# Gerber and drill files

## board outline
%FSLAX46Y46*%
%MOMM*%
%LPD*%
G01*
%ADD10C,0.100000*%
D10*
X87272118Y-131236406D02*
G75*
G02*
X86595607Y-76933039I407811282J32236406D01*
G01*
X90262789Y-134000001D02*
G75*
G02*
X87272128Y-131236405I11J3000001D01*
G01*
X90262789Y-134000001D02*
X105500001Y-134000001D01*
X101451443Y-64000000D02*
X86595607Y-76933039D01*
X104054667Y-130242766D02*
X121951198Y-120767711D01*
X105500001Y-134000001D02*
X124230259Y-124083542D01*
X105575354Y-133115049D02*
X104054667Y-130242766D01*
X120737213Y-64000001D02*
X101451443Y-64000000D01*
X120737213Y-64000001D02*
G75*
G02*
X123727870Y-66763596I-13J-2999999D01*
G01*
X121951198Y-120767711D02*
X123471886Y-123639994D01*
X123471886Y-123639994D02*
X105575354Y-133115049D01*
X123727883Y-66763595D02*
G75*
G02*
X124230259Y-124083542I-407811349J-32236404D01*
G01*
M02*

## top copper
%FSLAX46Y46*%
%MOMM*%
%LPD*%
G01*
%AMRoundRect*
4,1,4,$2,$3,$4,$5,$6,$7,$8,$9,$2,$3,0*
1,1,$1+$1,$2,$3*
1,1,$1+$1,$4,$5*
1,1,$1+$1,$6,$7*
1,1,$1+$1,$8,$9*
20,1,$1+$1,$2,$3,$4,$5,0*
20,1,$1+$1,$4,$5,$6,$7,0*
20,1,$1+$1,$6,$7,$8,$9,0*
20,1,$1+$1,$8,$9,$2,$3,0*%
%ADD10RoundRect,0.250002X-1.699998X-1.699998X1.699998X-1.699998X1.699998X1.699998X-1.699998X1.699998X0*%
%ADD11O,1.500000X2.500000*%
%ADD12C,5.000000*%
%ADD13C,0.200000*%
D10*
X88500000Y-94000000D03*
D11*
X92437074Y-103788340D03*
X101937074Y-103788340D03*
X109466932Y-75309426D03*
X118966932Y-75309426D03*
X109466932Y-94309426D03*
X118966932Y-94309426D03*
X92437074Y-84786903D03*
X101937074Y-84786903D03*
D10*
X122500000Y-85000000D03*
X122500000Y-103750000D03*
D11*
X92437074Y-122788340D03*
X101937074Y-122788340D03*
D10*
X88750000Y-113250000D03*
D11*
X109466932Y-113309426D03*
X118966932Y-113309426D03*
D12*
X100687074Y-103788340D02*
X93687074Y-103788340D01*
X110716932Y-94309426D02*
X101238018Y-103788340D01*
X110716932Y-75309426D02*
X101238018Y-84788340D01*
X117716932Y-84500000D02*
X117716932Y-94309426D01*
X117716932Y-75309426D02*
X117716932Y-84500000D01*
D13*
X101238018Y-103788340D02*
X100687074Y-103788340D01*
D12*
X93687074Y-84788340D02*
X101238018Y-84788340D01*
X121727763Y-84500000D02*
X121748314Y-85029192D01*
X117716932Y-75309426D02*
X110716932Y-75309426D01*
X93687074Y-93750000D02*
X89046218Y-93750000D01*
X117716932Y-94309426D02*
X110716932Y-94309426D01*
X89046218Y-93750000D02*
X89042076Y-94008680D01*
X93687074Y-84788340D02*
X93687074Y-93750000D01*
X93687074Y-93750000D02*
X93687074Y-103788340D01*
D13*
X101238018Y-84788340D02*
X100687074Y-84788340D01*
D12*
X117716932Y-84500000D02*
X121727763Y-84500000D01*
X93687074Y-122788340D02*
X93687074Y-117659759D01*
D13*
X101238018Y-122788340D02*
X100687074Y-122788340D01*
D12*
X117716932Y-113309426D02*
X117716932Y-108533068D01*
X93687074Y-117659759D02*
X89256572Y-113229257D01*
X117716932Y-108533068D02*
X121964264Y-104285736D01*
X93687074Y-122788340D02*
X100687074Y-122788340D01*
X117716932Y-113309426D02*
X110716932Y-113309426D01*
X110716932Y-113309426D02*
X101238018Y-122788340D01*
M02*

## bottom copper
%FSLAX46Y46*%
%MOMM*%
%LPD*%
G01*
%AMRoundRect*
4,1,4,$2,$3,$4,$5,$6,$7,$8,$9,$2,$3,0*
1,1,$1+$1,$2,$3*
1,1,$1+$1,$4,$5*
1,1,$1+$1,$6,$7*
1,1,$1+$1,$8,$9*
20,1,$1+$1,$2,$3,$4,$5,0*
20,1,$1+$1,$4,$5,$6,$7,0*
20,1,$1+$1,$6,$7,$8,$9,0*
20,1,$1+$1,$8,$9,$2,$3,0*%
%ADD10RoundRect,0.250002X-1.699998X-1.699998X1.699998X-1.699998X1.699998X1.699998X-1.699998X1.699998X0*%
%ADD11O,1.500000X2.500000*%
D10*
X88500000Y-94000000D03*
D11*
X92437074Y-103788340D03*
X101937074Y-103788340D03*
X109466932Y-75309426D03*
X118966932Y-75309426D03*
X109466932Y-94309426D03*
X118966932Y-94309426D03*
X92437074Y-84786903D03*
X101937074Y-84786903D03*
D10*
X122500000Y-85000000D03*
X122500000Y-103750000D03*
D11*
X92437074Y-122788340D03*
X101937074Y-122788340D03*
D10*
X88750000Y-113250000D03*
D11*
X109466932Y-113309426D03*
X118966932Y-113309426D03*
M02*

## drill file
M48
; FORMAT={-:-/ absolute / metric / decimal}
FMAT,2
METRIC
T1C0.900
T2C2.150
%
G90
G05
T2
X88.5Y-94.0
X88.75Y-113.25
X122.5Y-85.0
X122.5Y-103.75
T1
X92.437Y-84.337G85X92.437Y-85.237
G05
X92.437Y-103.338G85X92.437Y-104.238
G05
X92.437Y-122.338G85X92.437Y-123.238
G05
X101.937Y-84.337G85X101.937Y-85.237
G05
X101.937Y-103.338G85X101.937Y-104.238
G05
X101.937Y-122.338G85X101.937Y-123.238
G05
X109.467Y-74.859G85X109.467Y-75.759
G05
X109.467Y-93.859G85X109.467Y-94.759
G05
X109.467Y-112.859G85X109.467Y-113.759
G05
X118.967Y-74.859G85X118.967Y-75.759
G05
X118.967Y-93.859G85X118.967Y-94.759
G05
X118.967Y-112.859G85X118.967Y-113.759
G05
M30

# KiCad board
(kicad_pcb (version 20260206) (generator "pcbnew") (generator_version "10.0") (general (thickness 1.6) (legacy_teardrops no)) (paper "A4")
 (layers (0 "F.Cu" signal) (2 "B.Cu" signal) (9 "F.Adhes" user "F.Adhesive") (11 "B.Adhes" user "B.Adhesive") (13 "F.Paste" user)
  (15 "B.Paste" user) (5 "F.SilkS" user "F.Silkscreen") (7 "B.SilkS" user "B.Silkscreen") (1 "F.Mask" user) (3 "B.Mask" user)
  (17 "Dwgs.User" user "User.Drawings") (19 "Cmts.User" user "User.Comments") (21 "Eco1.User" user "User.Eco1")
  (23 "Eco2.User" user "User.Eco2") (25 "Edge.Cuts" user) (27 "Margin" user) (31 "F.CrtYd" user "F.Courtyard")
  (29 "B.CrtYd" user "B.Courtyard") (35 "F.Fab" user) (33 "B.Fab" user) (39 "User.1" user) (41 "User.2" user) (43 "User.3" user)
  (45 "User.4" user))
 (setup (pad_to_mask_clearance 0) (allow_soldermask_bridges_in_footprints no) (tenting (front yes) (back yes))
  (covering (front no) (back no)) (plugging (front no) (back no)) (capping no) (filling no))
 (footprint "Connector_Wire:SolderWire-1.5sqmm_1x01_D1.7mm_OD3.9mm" (layer "F.Cu") (at 88.5 94)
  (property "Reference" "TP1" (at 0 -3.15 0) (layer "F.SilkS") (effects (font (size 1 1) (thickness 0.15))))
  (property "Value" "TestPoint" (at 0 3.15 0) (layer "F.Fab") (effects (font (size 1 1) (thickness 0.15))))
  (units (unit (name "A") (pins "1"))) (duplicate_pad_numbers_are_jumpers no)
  (pad "1" thru_hole roundrect (at 0 0) (size 3.9 3.9) (drill 2.15) (layers "*.Cu" "*.Mask") (remove_unused_layers no)
   (roundrect_rratio 0.064103) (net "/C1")))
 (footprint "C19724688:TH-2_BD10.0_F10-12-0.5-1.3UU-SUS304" (layer "F.Cu") (at 97.187074 103.78834)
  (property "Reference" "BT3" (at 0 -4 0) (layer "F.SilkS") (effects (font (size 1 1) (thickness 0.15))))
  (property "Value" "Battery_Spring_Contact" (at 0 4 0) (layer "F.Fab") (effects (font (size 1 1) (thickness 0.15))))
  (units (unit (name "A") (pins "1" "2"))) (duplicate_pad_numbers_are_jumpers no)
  (pad "1" thru_hole oval (at -4.75 0) (size 1.5 2.5) (drill oval 0.900024 1.799996) (layers "*.Cu" "*.Mask") (remove_unused_layers no)
   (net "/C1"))
  (pad "2" thru_hole oval (at 4.75 0) (size 1.5 2.5) (drill oval 0.900024 1.799996) (layers "*.Cu" "*.Mask") (remove_unused_layers no)
   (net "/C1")))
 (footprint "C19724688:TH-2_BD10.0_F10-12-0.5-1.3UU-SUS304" (layer "F.Cu") (at 114.216932 75.309426)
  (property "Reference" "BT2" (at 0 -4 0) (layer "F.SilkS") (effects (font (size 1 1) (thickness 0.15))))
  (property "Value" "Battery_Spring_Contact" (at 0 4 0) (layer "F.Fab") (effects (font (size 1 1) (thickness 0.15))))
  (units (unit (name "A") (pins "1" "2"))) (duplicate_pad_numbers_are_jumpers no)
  (pad "1" thru_hole oval (at -4.75 0) (size 1.5 2.5) (drill oval 0.900024 1.799996) (layers "*.Cu" "*.Mask") (remove_unused_layers no)
   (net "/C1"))
  (pad "2" thru_hole oval (at 4.75 0) (size 1.5 2.5) (drill oval 0.900024 1.799996) (layers "*.Cu" "*.Mask") (remove_unused_layers no)
   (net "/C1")))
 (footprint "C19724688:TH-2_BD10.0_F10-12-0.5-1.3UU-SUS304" (layer "F.Cu") (at 114.216932 94.309426)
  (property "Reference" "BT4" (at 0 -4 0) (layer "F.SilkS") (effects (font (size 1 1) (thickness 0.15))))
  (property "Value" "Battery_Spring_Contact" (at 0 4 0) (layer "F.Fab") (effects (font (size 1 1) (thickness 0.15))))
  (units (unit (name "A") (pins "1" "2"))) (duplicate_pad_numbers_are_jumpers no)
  (pad "1" thru_hole oval (at -4.75 0) (size 1.5 2.5) (drill oval 0.900024 1.799996) (layers "*.Cu" "*.Mask") (remove_unused_layers no)
   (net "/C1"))
  (pad "2" thru_hole oval (at 4.75 0) (size 1.5 2.5) (drill oval 0.900024 1.799996) (layers "*.Cu" "*.Mask") (remove_unused_layers no)
   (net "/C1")))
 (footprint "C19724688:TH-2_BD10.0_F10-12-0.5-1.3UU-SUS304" (layer "F.Cu") (at 97.187074 84.786903)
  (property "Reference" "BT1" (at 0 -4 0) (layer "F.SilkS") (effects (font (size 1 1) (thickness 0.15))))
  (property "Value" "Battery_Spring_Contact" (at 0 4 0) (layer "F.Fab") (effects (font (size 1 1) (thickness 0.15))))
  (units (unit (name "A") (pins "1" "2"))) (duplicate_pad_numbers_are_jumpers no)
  (pad "1" thru_hole oval (at -4.75 0) (size 1.5 2.5) (drill oval 0.900024 1.799996) (layers "*.Cu" "*.Mask") (remove_unused_layers no)
   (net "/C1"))
  (pad "2" thru_hole oval (at 4.75 0) (size 1.5 2.5) (drill oval 0.900024 1.799996) (layers "*.Cu" "*.Mask") (remove_unused_layers no)
   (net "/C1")))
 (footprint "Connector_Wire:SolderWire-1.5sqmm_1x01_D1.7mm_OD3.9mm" (layer "F.Cu") (at 122.5 85)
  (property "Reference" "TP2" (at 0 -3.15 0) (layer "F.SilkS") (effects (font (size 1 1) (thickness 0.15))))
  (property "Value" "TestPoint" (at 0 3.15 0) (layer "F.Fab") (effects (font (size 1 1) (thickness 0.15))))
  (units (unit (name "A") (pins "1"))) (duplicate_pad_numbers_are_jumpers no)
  (pad "1" thru_hole roundrect (at 0 0) (size 3.9 3.9) (drill 2.15) (layers "*.Cu" "*.Mask") (remove_unused_layers no)
   (roundrect_rratio 0.064103) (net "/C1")))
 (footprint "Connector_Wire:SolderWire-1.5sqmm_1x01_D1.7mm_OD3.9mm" (layer "F.Cu") (at 122.5 103.75)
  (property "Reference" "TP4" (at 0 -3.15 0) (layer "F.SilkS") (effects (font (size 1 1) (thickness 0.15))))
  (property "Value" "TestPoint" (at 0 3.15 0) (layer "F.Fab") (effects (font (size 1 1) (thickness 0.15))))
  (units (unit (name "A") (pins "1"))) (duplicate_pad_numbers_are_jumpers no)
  (pad "1" thru_hole roundrect (at 0 0) (size 3.9 3.9) (drill 2.15) (layers "*.Cu" "*.Mask") (remove_unused_layers no)
   (roundrect_rratio 0.064103) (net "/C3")))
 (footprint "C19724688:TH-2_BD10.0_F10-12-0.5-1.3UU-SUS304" (layer "F.Cu") (at 97.187074 122.78834)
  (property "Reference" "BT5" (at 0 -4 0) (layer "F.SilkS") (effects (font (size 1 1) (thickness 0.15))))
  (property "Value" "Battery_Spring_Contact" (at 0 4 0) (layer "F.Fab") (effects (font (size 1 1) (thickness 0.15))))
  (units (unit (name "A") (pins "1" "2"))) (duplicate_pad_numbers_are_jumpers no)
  (pad "1" thru_hole oval (at -4.75 0) (size 1.5 2.5) (drill oval 0.900024 1.799996) (layers "*.Cu" "*.Mask") (remove_unused_layers no)
   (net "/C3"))
  (pad "2" thru_hole oval (at 4.75 0) (size 1.5 2.5) (drill oval 0.900024 1.799996) (layers "*.Cu" "*.Mask") (remove_unused_layers no)
   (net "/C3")))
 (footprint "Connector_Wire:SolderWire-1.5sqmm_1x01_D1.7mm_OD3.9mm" (layer "F.Cu") (at 88.75 113.25)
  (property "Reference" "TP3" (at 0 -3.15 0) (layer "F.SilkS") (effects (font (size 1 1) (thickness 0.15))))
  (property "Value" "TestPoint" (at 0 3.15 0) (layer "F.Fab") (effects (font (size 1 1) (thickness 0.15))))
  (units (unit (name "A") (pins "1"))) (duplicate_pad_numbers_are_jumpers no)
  (pad "1" thru_hole roundrect (at 0 0) (size 3.9 3.9) (drill 2.15) (layers "*.Cu" "*.Mask") (remove_unused_layers no)
   (roundrect_rratio 0.064103) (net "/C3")))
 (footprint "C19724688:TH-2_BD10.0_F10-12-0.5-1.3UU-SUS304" (layer "F.Cu") (at 114.216932 113.309426)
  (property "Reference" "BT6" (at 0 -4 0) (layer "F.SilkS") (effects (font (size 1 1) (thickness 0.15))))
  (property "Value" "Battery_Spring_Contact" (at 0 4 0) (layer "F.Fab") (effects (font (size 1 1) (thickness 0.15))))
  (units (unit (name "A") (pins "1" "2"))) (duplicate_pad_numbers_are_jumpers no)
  (pad "1" thru_hole oval (at -4.75 0) (size 1.5 2.5) (drill oval 0.900024 1.799996) (layers "*.Cu" "*.Mask") (remove_unused_layers no)
   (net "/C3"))
  (pad "2" thru_hole oval (at 4.75 0) (size 1.5 2.5) (drill oval 0.900024 1.799996) (layers "*.Cu" "*.Mask") (remove_unused_layers no)
   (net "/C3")))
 (gr_arc (start 87.272118 131.236406) (mid 86.031742 104.095961) (end 86.595607 76.933039) (stroke (width 0.1) (type default))
  (layer "Edge.Cuts"))
 (gr_arc (start 90.262789 134.000001) (mid 88.226767 133.203318) (end 87.272118 131.236406) (stroke (width 0.1) (type default))
  (layer "Edge.Cuts"))
 (gr_line (start 90.262789 134.000001) (end 105.500001 134.000001) (stroke (width 0.1) (type default)) (layer "Edge.Cuts"))
 (gr_line (start 101.451443 64) (end 86.595607 76.933039) (stroke (width 0.1) (type default)) (layer "Edge.Cuts"))
 (gr_line (start 104.054667 130.242766) (end 121.951198 120.767711) (stroke (width 0.1) (type default)) (layer "Edge.Cuts"))
 (gr_line (start 105.500001 134.000001) (end 124.230259 124.083542) (stroke (width 0.1) (type default)) (layer "Edge.Cuts"))
 (gr_line (start 105.575354 133.115049) (end 104.054667 130.242766) (stroke (width 0.1) (type default)) (layer "Edge.Cuts"))
 (gr_line (start 120.737213 64.000001) (end 101.451443 64) (stroke (width 0.1) (type default)) (layer "Edge.Cuts"))
 (gr_arc (start 120.737213 64.000001) (mid 122.773235 64.796684) (end 123.727883 66.763595) (stroke (width 0.1) (type default))
  (layer "Edge.Cuts"))
 (gr_line (start 121.951198 120.767711) (end 123.471886 123.639994) (stroke (width 0.1) (type default)) (layer "Edge.Cuts"))
 (gr_line (start 123.471886 123.639994) (end 105.575354 133.115049) (stroke (width 0.1) (type default)) (layer "Edge.Cuts"))
 (gr_arc (start 123.727883 66.763595) (mid 124.984289 95.414758) (end 124.230259 124.083542) (stroke (width 0.1) (type default))
  (layer "Edge.Cuts"))
 (segment (start 100.687074 103.78834) (end 93.687074 103.78834) (width 5) (layer "F.Cu") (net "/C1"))
 (segment (start 110.716932 94.309426) (end 101.238018 103.78834) (width 5) (layer "F.Cu") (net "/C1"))
 (segment (start 110.716932 75.309426) (end 101.238018 84.78834) (width 5) (layer "F.Cu") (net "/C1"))
 (segment (start 117.716932 84.5) (end 117.716932 94.309426) (width 5) (layer "F.Cu") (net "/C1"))
 (segment (start 117.716932 75.309426) (end 117.716932 84.5) (width 5) (layer "F.Cu") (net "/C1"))
 (segment (start 101.238018 103.78834) (end 100.687074 103.78834) (width 0.2) (layer "F.Cu") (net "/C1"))
 (segment (start 93.687074 84.78834) (end 101.238018 84.78834) (width 5) (layer "F.Cu") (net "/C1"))
 (segment (start 121.727763 84.5) (end 121.748314 85.029192) (width 5) (layer "F.Cu") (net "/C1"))
 (segment (start 117.716932 75.309426) (end 110.716932 75.309426) (width 5) (layer "F.Cu") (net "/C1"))
 (segment (start 93.687074 93.75) (end 89.046218 93.75) (width 5) (layer "F.Cu") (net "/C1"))
 (segment (start 117.716932 94.309426) (end 110.716932 94.309426) (width 5) (layer "F.Cu") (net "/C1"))
 (segment (start 89.046218 93.75) (end 89.042076 94.00868) (width 5) (layer "F.Cu") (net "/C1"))
 (segment (start 93.687074 84.78834) (end 93.687074 93.75) (width 5) (layer "F.Cu") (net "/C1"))
 (segment (start 93.687074 93.75) (end 93.687074 103.78834) (width 5) (layer "F.Cu") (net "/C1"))
 (segment (start 101.238018 84.78834) (end 100.687074 84.78834) (width 0.2) (layer "F.Cu") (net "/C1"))
 (segment (start 117.716932 84.5) (end 121.727763 84.5) (width 5) (layer "F.Cu") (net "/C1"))
 (segment (start 93.687074 122.78834) (end 93.687074 117.659759) (width 5) (layer "F.Cu") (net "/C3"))
 (segment (start 101.238018 122.78834) (end 100.687074 122.78834) (width 0.2) (layer "F.Cu") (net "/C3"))
 (segment (start 117.716932 113.309426) (end 117.716932 108.533068) (width 5) (layer "F.Cu") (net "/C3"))
 (segment (start 93.687074 117.659759) (end 89.256572 113.229257) (width 5) (layer "F.Cu") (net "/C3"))
 (segment (start 117.716932 108.533068) (end 121.964264 104.285736) (width 5) (layer "F.Cu") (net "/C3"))
 (segment (start 93.687074 122.78834) (end 100.687074 122.78834) (width 5) (layer "F.Cu") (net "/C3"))
 (segment (start 117.716932 113.309426) (end 110.716932 113.309426) (width 5) (layer "F.Cu") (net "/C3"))
 (segment (start 110.716932 113.309426) (end 101.238018 122.78834) (width 5) (layer "F.Cu") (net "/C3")))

